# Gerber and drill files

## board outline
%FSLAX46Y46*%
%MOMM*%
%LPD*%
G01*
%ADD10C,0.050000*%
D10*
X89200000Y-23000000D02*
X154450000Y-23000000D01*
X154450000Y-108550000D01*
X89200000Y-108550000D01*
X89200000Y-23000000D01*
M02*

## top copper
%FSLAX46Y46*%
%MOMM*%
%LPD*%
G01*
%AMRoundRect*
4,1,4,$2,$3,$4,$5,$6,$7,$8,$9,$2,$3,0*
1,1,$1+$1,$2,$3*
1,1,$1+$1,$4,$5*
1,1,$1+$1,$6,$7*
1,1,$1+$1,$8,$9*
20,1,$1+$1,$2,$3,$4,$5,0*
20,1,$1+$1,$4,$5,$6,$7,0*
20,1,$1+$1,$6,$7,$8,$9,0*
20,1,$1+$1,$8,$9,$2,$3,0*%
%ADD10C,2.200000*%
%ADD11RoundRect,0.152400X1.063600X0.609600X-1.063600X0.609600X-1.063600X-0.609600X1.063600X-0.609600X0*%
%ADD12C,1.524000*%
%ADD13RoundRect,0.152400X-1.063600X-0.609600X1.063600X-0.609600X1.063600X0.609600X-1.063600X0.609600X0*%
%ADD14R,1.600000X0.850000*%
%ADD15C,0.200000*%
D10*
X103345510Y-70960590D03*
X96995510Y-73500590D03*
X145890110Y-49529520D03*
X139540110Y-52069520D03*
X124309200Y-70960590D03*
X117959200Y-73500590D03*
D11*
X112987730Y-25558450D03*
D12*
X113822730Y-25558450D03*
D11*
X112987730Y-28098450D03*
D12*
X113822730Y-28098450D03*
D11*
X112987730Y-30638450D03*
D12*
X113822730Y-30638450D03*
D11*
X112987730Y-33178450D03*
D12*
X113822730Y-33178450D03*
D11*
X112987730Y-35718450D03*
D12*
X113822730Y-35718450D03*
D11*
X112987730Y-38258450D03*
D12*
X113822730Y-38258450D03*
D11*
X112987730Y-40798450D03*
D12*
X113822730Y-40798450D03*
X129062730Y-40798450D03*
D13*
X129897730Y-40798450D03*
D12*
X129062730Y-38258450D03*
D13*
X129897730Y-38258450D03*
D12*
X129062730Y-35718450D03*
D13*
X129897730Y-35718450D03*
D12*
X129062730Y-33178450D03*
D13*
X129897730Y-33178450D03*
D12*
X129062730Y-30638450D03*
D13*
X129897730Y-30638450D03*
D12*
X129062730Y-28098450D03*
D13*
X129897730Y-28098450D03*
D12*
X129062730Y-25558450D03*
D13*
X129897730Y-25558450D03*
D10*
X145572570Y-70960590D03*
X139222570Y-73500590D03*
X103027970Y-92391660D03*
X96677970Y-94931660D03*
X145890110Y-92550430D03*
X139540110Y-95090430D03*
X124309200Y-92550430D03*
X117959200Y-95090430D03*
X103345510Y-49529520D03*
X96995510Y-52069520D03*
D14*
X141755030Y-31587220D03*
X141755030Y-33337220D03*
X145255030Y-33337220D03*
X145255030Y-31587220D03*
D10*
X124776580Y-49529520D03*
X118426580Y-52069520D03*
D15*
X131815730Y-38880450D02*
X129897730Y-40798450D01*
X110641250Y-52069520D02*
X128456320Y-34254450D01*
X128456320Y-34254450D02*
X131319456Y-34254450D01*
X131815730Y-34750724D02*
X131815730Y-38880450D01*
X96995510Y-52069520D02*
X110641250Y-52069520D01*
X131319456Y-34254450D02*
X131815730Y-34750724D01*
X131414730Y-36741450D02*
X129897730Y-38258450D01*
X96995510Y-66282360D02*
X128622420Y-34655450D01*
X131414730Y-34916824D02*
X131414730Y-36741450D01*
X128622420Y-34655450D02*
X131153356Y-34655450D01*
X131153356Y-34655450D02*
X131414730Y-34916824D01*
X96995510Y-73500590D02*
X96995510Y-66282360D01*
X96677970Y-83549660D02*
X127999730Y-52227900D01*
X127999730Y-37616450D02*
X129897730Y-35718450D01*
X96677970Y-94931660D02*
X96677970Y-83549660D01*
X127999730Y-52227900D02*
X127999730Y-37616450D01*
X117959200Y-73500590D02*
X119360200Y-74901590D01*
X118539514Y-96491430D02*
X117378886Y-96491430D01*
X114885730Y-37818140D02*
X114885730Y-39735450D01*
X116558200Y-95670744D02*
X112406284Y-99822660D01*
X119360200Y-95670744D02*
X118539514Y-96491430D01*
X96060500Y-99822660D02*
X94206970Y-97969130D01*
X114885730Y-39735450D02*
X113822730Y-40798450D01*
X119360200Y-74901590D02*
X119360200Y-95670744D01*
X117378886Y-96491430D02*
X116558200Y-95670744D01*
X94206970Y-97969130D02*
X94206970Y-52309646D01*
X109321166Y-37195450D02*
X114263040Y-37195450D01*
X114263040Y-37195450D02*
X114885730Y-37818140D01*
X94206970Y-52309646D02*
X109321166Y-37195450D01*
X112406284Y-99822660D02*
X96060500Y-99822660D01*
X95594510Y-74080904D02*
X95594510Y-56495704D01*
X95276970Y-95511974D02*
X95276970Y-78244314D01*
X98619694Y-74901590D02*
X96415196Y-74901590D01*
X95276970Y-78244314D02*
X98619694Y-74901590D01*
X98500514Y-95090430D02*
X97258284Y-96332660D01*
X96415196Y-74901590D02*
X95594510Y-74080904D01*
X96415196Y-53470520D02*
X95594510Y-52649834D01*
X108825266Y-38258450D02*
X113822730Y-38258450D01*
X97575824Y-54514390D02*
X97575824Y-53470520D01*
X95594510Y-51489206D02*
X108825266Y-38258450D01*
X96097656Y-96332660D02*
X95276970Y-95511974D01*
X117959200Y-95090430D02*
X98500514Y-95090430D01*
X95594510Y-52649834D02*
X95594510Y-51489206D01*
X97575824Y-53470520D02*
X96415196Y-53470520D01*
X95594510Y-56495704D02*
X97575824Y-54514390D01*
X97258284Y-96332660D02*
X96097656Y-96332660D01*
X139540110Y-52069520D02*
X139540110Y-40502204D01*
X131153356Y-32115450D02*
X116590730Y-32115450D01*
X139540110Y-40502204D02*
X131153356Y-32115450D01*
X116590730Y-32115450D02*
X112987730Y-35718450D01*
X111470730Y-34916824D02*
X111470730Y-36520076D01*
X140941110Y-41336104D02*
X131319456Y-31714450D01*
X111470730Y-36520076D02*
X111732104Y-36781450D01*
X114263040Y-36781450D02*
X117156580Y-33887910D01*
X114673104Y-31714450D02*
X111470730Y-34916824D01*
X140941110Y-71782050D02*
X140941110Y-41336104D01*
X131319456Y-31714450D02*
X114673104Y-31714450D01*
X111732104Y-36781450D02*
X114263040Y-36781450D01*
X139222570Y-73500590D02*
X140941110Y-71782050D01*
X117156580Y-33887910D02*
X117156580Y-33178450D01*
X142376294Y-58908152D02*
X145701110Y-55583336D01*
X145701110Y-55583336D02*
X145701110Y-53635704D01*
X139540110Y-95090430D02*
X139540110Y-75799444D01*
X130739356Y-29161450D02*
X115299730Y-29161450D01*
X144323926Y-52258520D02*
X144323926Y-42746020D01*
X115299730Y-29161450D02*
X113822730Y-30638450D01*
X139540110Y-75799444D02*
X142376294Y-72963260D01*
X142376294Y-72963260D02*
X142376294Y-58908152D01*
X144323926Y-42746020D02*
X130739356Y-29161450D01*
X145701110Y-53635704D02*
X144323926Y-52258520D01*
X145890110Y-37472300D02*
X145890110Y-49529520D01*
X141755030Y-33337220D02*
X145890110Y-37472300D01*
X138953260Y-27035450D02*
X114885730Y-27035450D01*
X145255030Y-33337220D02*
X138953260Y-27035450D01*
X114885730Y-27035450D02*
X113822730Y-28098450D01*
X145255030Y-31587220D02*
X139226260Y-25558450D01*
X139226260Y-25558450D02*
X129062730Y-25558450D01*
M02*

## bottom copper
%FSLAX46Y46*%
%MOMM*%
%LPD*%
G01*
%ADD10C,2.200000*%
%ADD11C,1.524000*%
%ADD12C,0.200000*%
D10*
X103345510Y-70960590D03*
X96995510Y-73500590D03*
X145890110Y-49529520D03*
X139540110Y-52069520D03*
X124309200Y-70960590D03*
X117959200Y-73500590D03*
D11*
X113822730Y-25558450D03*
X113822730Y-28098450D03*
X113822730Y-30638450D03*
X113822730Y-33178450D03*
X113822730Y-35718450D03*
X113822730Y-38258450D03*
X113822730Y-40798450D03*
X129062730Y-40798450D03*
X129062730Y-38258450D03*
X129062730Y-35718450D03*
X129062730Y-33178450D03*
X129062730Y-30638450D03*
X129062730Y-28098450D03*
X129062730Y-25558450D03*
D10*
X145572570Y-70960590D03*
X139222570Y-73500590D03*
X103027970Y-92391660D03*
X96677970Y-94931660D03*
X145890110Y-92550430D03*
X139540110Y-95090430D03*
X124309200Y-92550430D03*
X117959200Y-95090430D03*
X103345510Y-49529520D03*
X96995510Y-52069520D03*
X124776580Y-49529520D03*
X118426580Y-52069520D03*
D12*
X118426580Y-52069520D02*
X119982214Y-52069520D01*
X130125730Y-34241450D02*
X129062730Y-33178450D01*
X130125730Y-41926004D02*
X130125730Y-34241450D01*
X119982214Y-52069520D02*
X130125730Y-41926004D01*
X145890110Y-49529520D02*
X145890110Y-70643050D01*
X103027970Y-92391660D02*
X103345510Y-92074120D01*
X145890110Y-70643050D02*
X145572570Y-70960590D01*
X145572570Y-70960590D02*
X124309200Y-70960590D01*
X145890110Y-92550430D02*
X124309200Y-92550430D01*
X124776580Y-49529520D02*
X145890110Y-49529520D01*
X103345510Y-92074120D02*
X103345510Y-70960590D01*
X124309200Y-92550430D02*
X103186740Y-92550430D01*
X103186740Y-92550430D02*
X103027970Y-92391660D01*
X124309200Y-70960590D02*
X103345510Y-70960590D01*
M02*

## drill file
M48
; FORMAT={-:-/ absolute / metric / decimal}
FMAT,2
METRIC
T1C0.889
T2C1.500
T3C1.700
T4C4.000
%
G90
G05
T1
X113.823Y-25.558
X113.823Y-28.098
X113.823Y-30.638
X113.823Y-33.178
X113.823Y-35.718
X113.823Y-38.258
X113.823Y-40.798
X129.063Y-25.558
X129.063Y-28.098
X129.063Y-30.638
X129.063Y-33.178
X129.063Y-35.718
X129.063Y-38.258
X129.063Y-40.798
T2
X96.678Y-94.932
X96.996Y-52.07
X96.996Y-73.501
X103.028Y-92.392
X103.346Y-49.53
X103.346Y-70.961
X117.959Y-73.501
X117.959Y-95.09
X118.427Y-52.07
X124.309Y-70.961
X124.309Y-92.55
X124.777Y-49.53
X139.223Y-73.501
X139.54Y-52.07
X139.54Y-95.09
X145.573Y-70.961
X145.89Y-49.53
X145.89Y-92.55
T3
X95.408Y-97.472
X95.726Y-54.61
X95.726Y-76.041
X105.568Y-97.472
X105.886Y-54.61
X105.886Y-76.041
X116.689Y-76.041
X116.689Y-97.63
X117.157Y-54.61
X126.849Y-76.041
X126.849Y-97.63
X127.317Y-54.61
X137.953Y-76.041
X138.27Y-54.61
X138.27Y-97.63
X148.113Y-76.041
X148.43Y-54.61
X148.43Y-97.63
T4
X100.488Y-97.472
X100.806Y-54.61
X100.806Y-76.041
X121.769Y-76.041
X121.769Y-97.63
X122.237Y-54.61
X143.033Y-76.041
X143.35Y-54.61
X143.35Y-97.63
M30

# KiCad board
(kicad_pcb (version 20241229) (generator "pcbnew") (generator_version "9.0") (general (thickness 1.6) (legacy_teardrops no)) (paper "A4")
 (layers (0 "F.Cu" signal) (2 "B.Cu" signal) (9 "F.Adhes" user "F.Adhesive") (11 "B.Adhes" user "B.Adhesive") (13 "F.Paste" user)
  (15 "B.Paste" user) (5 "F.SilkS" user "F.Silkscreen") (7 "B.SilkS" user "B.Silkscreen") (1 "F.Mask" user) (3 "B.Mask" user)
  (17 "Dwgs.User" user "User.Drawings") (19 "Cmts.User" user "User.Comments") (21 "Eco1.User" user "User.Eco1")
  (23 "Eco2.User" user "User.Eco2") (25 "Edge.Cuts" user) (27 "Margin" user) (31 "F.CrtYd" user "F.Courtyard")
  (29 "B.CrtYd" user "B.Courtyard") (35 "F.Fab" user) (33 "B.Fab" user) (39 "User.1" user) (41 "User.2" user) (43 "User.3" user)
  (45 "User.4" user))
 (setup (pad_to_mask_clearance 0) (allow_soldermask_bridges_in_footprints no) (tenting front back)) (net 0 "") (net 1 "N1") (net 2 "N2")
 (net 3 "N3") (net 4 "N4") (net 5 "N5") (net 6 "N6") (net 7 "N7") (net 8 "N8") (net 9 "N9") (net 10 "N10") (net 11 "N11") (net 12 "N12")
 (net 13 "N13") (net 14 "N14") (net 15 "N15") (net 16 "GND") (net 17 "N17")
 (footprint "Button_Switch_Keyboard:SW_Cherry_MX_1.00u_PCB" (layer "F.Cu") (at 103.34551 70.96059)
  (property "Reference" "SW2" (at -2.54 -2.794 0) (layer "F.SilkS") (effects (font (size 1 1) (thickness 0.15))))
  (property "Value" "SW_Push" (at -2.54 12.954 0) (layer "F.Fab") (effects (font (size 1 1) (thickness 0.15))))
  (pad "" np_thru_hole circle (at -7.62 5.08) (size 1.7 1.7) (drill 1.7) (layers "*.Cu" "*.Mask"))
  (pad "" np_thru_hole circle (at -2.54 5.08) (size 4 4) (drill 4) (layers "*.Cu" "*.Mask"))
  (pad "" np_thru_hole circle (at 2.54 5.08) (size 1.7 1.7) (drill 1.7) (layers "*.Cu" "*.Mask"))
  (pad "1" thru_hole circle (at 0 0) (size 2.2 2.2) (drill 1.5) (layers "*.Cu" "*.Mask") (remove_unused_layers no) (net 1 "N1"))
  (pad "2" thru_hole circle (at -6.35 2.54) (size 2.2 2.2) (drill 1.5) (layers "*.Cu" "*.Mask") (remove_unused_layers no) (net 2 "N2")))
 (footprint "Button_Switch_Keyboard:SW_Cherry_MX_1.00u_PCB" (layer "F.Cu") (at 145.89011 49.52952)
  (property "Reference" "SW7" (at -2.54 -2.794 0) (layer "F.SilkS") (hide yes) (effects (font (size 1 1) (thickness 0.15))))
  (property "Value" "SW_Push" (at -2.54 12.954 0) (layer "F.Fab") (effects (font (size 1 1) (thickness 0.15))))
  (pad "" np_thru_hole circle (at -7.62 5.08) (size 1.7 1.7) (drill 1.7) (layers "*.Cu" "*.Mask"))
  (pad "" np_thru_hole circle (at -2.54 5.08) (size 4 4) (drill 4) (layers "*.Cu" "*.Mask"))
  (pad "" np_thru_hole circle (at 2.54 5.08) (size 1.7 1.7) (drill 1.7) (layers "*.Cu" "*.Mask"))
  (pad "1" thru_hole circle (at 0 0) (size 2.2 2.2) (drill 1.5) (layers "*.Cu" "*.Mask") (remove_unused_layers no) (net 1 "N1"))
  (pad "2" thru_hole circle (at -6.35 2.54) (size 2.2 2.2) (drill 1.5) (layers "*.Cu" "*.Mask") (remove_unused_layers no) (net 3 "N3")))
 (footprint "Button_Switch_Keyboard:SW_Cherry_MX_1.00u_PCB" (layer "F.Cu") (at 124.3092 70.96059)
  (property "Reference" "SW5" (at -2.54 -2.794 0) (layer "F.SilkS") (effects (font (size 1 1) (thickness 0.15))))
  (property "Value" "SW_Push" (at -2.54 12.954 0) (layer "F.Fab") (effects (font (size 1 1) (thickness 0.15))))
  (pad "" np_thru_hole circle (at -7.62 5.08) (size 1.7 1.7) (drill 1.7) (layers "*.Cu" "*.Mask"))
  (pad "" np_thru_hole circle (at -2.54 5.08) (size 4 4) (drill 4) (layers "*.Cu" "*.Mask"))
  (pad "" np_thru_hole circle (at 2.54 5.08) (size 1.7 1.7) (drill 1.7) (layers "*.Cu" "*.Mask"))
  (pad "1" thru_hole circle (at 0 0) (size 2.2 2.2) (drill 1.5) (layers "*.Cu" "*.Mask") (remove_unused_layers no) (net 1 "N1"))
  (pad "2" thru_hole circle (at -6.35 2.54) (size 2.2 2.2) (drill 1.5) (layers "*.Cu" "*.Mask") (remove_unused_layers no) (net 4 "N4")))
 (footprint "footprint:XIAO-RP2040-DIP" (layer "F.Cu") (at 121.44273 33.17845)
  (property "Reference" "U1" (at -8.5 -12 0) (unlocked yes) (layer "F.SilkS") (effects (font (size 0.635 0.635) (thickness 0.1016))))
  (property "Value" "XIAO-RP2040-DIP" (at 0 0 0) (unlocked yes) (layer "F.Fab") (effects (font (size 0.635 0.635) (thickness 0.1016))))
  (pad "1" smd roundrect (at -8.455 -7.62 180) (size 2.432 1.524) (layers "F.Cu" "F.Mask") (roundrect_rratio 0.1) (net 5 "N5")
   (thermal_bridge_angle 45))
  (pad "1" thru_hole circle (at -7.62 -7.62 180) (size 1.524 1.524) (drill 0.889) (layers "*.Cu" "*.Mask") (remove_unused_layers no)
   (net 5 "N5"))
  (pad "2" smd roundrect (at -8.455 -5.08 180) (size 2.432 1.524) (layers "F.Cu" "F.Mask") (roundrect_rratio 0.1) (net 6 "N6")
   (thermal_bridge_angle 45))
  (pad "2" thru_hole circle (at -7.62 -5.08 180) (size 1.524 1.524) (drill 0.889) (layers "*.Cu" "*.Mask") (remove_unused_layers no)
   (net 6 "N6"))
  (pad "3" smd roundrect (at -8.455 -2.54 180) (size 2.432 1.524) (layers "F.Cu" "F.Mask") (roundrect_rratio 0.1) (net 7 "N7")
   (thermal_bridge_angle 45))
  (pad "3" thru_hole circle (at -7.62 -2.54 180) (size 1.524 1.524) (drill 0.889) (layers "*.Cu" "*.Mask") (remove_unused_layers no)
   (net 7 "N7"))
  (pad "4" smd roundrect (at -8.455 0 180) (size 2.432 1.524) (layers "F.Cu" "F.Mask") (roundrect_rratio 0.1) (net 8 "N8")
   (thermal_bridge_angle 45))
  (pad "4" thru_hole circle (at -7.62 0 180) (size 1.524 1.524) (drill 0.889) (layers "*.Cu" "*.Mask") (remove_unused_layers no)
   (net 8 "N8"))
  (pad "5" smd roundrect (at -8.455 2.54 180) (size 2.432 1.524) (layers "F.Cu" "F.Mask") (roundrect_rratio 0.1) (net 3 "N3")
   (thermal_bridge_angle 45))
  (pad "5" thru_hole circle (at -7.62 2.54 180) (size 1.524 1.524) (drill 0.889) (layers "*.Cu" "*.Mask") (remove_unused_layers no)
   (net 3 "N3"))
  (pad "6" smd roundrect (at -8.455 5.08 180) (size 2.432 1.524) (layers "F.Cu" "F.Mask") (roundrect_rratio 0.1) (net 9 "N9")
   (thermal_bridge_angle 45))
  (pad "6" thru_hole circle (at -7.62 5.08 180) (size 1.524 1.524) (drill 0.889) (layers "*.Cu" "*.Mask") (remove_unused_layers no)
   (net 9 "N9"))
  (pad "7" smd roundrect (at -8.455 7.62 180) (size 2.432 1.524) (layers "F.Cu" "F.Mask") (roundrect_rratio 0.1) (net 4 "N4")
   (thermal_bridge_angle 45))
  (pad "7" thru_hole circle (at -7.62 7.62 180) (size 1.524 1.524) (drill 0.889) (layers "*.Cu" "*.Mask") (remove_unused_layers no)
   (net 4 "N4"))
  (pad "8" thru_hole circle (at 7.62 7.62) (size 1.524 1.524) (drill 0.889) (layers "*.Cu" "*.Mask") (remove_unused_layers no)
   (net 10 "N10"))
  (pad "8" smd roundrect (at 8.455 7.62) (size 2.432 1.524) (layers "F.Cu" "F.Mask") (roundrect_rratio 0.1) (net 10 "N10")
   (thermal_bridge_angle 45))
  (pad "9" thru_hole circle (at 7.62 5.08) (size 1.524 1.524) (drill 0.889) (layers "*.Cu" "*.Mask") (remove_unused_layers no) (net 2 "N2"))
  (pad "9" smd roundrect (at 8.455 5.08) (size 2.432 1.524) (layers "F.Cu" "F.Mask") (roundrect_rratio 0.1) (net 2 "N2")
   (thermal_bridge_angle 45))
  (pad "10" thru_hole circle (at 7.62 2.54) (size 1.524 1.524) (drill 0.889) (layers "*.Cu" "*.Mask") (remove_unused_layers no)
   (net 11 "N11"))
  (pad "10" smd roundrect (at 8.455 2.54) (size 2.432 1.524) (layers "F.Cu" "F.Mask") (roundrect_rratio 0.1) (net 11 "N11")
   (thermal_bridge_angle 45))
  (pad "11" thru_hole circle (at 7.62 0) (size 1.524 1.524) (drill 0.889) (layers "*.Cu" "*.Mask") (remove_unused_layers no) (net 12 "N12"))
  (pad "11" smd roundrect (at 8.455 0) (size 2.432 1.524) (layers "F.Cu" "F.Mask") (roundrect_rratio 0.1) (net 12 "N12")
   (thermal_bridge_angle 45))
  (pad "12" thru_hole circle (at 7.62 -2.54) (size 1.524 1.524) (drill 0.889) (layers "*.Cu" "*.Mask") (remove_unused_layers no)
   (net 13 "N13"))
  (pad "12" smd roundrect (at 8.455 -2.54) (size 2.432 1.524) (layers "F.Cu" "F.Mask") (roundrect_rratio 0.1) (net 13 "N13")
   (thermal_bridge_angle 45))
  (pad "13" thru_hole circle (at 7.62 -5.08) (size 1.524 1.524) (drill 0.889) (layers "*.Cu" "*.Mask") (remove_unused_layers no)
   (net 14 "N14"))
  (pad "13" smd roundrect (at 8.455 -5.08) (size 2.432 1.524) (layers "F.Cu" "F.Mask") (roundrect_rratio 0.1) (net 14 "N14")
   (thermal_bridge_angle 45))
  (pad "14" thru_hole circle (at 7.62 -7.62) (size 1.524 1.524) (drill 0.889) (layers "*.Cu" "*.Mask") (remove_unused_layers no)
   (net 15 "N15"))
  (pad "14" smd roundrect (at 8.455 -7.62) (size 2.432 1.524) (layers "F.Cu" "F.Mask") (roundrect_rratio 0.1) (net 15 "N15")
   (thermal_bridge_angle 45)))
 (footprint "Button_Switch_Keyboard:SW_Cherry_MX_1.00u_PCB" (layer "F.Cu") (at 145.57257 70.96059)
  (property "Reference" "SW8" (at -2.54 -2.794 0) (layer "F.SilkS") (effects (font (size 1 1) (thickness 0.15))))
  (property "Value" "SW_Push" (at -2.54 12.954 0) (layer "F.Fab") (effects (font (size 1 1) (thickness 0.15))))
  (pad "" np_thru_hole circle (at -7.62 5.08) (size 1.7 1.7) (drill 1.7) (layers "*.Cu" "*.Mask"))
  (pad "" np_thru_hole circle (at -2.54 5.08) (size 4 4) (drill 4) (layers "*.Cu" "*.Mask"))
  (pad "" np_thru_hole circle (at 2.54 5.08) (size 1.7 1.7) (drill 1.7) (layers "*.Cu" "*.Mask"))
  (pad "1" thru_hole circle (at 0 0) (size 2.2 2.2) (drill 1.5) (layers "*.Cu" "*.Mask") (remove_unused_layers no) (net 1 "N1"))
  (pad "2" thru_hole circle (at -6.35 2.54) (size 2.2 2.2) (drill 1.5) (layers "*.Cu" "*.Mask") (remove_unused_layers no) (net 8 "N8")))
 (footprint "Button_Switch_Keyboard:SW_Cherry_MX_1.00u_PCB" (layer "F.Cu") (at 103.02797 92.39166)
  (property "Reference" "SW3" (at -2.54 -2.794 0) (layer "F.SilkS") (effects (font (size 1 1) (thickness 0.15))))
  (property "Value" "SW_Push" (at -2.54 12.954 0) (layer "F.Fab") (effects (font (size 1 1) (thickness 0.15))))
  (pad "" np_thru_hole circle (at -7.62 5.08) (size 1.7 1.7) (drill 1.7) (layers "*.Cu" "*.Mask"))
  (pad "" np_thru_hole circle (at -2.54 5.08) (size 4 4) (drill 4) (layers "*.Cu" "*.Mask"))
  (pad "" np_thru_hole circle (at 2.54 5.08) (size 1.7 1.7) (drill 1.7) (layers "*.Cu" "*.Mask"))
  (pad "1" thru_hole circle (at 0 0) (size 2.2 2.2) (drill 1.5) (layers "*.Cu" "*.Mask") (remove_unused_layers no) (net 1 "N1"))
  (pad "2" thru_hole circle (at -6.35 2.54) (size 2.2 2.2) (drill 1.5) (layers "*.Cu" "*.Mask") (remove_unused_layers no) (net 11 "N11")))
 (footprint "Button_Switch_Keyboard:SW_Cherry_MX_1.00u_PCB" (layer "F.Cu") (at 145.89011 92.55043)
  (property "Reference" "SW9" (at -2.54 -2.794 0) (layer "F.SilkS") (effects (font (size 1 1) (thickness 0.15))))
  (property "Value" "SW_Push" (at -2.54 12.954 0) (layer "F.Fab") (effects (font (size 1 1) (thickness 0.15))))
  (pad "" np_thru_hole circle (at -7.62 5.08) (size 1.7 1.7) (drill 1.7) (layers "*.Cu" "*.Mask"))
  (pad "" np_thru_hole circle (at -2.54 5.08) (size 4 4) (drill 4) (layers "*.Cu" "*.Mask"))
  (pad "" np_thru_hole circle (at 2.54 5.08) (size 1.7 1.7) (drill 1.7) (layers "*.Cu" "*.Mask"))
  (pad "1" thru_hole circle (at 0 0) (size 2.2 2.2) (drill 1.5) (layers "*.Cu" "*.Mask") (remove_unused_layers no) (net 1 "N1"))
  (pad "2" thru_hole circle (at -6.35 2.54) (size 2.2 2.2) (drill 1.5) (layers "*.Cu" "*.Mask") (remove_unused_layers no) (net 7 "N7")))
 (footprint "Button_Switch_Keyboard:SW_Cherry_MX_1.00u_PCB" (layer "F.Cu") (at 124.3092 92.55043)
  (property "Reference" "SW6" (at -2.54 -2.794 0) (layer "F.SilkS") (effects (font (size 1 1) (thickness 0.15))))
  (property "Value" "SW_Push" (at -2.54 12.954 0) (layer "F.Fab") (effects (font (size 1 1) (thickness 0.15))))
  (pad "" np_thru_hole circle (at -7.62 5.08) (size 1.7 1.7) (drill 1.7) (layers "*.Cu" "*.Mask"))
  (pad "" np_thru_hole circle (at -2.54 5.08) (size 4 4) (drill 4) (layers "*.Cu" "*.Mask"))
  (pad "" np_thru_hole circle (at 2.54 5.08) (size 1.7 1.7) (drill 1.7) (layers "*.Cu" "*.Mask"))
  (pad "1" thru_hole circle (at 0 0) (size 2.2 2.2) (drill 1.5) (layers "*.Cu" "*.Mask") (remove_unused_layers no) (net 1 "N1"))
  (pad "2" thru_hole circle (at -6.35 2.54) (size 2.2 2.2) (drill 1.5) (layers "*.Cu" "*.Mask") (remove_unused_layers no) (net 9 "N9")))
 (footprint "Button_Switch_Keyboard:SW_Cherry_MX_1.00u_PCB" (layer "F.Cu") (at 103.34551 49.52952)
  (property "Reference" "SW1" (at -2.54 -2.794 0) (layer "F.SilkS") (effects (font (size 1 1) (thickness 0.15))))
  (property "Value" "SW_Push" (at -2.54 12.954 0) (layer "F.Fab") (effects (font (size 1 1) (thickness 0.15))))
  (pad "" np_thru_hole circle (at -7.62 5.08) (size 1.7 1.7) (drill 1.7) (layers "*.Cu" "*.Mask"))
  (pad "" np_thru_hole circle (at -2.54 5.08) (size 4 4) (drill 4) (layers "*.Cu" "*.Mask"))
  (pad "" np_thru_hole circle (at 2.54 5.08) (size 1.7 1.7) (drill 1.7) (layers "*.Cu" "*.Mask"))
  (pad "1" thru_hole circle (at 0 0) (size 2.2 2.2) (drill 1.5) (layers "*.Cu" "*.Mask") (remove_unused_layers no) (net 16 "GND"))
  (pad "2" thru_hole circle (at -6.35 2.54) (size 2.2 2.2) (drill 1.5) (layers "*.Cu" "*.Mask") (remove_unused_layers no) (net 10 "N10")))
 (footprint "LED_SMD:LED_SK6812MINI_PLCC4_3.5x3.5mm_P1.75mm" (layer "F.Cu") (at 143.50503 32.46222)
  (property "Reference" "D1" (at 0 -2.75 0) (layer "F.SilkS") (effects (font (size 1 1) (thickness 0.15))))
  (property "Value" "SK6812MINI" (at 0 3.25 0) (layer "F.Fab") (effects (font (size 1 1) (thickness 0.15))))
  (pad "1" smd rect (at -1.75 -0.875) (size 1.6 0.85) (layers "F.Cu" "F.Mask" "F.Paste") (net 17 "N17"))
  (pad "2" smd rect (at -1.75 0.875) (size 1.6 0.85) (layers "F.Cu" "F.Mask" "F.Paste") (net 1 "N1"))
  (pad "3" smd rect (at 1.75 0.875) (size 1.6 0.85) (layers "F.Cu" "F.Mask" "F.Paste") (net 6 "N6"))
  (pad "4" smd rect (at 1.75 -0.875) (size 1.6 0.85) (layers "F.Cu" "F.Mask" "F.Paste") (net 15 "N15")))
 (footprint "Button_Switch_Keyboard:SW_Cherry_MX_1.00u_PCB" (layer "F.Cu") (at 124.77658 49.52952)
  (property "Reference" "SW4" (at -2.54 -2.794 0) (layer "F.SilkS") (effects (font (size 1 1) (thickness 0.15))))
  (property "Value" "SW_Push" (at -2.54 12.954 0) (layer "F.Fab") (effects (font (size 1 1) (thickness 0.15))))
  (pad "" np_thru_hole circle (at -7.62 5.08) (size 1.7 1.7) (drill 1.7) (layers "*.Cu" "*.Mask"))
  (pad "" np_thru_hole circle (at -2.54 5.08) (size 4 4) (drill 4) (layers "*.Cu" "*.Mask"))
  (pad "" np_thru_hole circle (at 2.54 5.08) (size 1.7 1.7) (drill 1.7) (layers "*.Cu" "*.Mask"))
  (pad "1" thru_hole circle (at 0 0) (size 2.2 2.2) (drill 1.5) (layers "*.Cu" "*.Mask") (remove_unused_layers no) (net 1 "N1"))
  (pad "2" thru_hole circle (at -6.35 2.54) (size 2.2 2.2) (drill 1.5) (layers "*.Cu" "*.Mask") (remove_unused_layers no) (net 12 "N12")))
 (gr_rect (start 89.2 23) (end 154.45 108.55) (stroke (width 0.05) (type default)) (fill no) (layer "Edge.Cuts"))
 (segment (start 131.81573 38.88045) (end 129.89773 40.79845) (width 0.2) (layer "F.Cu") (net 10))
 (segment (start 110.64125 52.06952) (end 128.45632 34.25445) (width 0.2) (layer "F.Cu") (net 10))
 (segment (start 128.45632 34.25445) (end 131.319456 34.25445) (width 0.2) (layer "F.Cu") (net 10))
 (segment (start 131.81573 34.750724) (end 131.81573 38.88045) (width 0.2) (layer "F.Cu") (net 10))
 (segment (start 96.99551 52.06952) (end 110.64125 52.06952) (width 0.2) (layer "F.Cu") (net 10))
 (segment (start 131.319456 34.25445) (end 131.81573 34.750724) (width 0.2) (layer "F.Cu") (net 10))
 (segment (start 131.41473 36.74145) (end 129.89773 38.25845) (width 0.2) (layer "F.Cu") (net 2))
 (segment (start 96.99551 66.28236) (end 128.62242 34.65545) (width 0.2) (layer "F.Cu") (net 2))
 (segment (start 131.41473 34.916824) (end 131.41473 36.74145) (width 0.2) (layer "F.Cu") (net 2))
 (segment (start 128.62242 34.65545) (end 131.153356 34.65545) (width 0.2) (layer "F.Cu") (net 2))
 (segment (start 131.153356 34.65545) (end 131.41473 34.916824) (width 0.2) (layer "F.Cu") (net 2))
 (segment (start 96.99551 73.50059) (end 96.99551 66.28236) (width 0.2) (layer "F.Cu") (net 2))
 (segment (start 96.67797 83.54966) (end 127.99973 52.2279) (width 0.2) (layer "F.Cu") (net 11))
 (segment (start 127.99973 37.61645) (end 129.89773 35.71845) (width 0.2) (layer "F.Cu") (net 11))
 (segment (start 96.67797 94.93166) (end 96.67797 83.54966) (width 0.2) (layer "F.Cu") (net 11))
 (segment (start 127.99973 52.2279) (end 127.99973 37.61645) (width 0.2) (layer "F.Cu") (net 11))
 (segment (start 118.42658 52.06952) (end 119.982214 52.06952) (width 0.2) (layer "B.Cu") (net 12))
 (segment (start 130.12573 34.24145) (end 129.06273 33.17845) (width 0.2) (layer "B.Cu") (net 12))
 (segment (start 130.12573 41.926004) (end 130.12573 34.24145) (width 0.2) (layer "B.Cu") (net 12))
 (segment (start 119.982214 52.06952) (end 130.12573 41.926004) (width 0.2) (layer "B.Cu") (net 12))
 (segment (start 117.9592 73.50059) (end 119.3602 74.90159) (width 0.2) (layer "F.Cu") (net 4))
 (segment (start 118.539514 96.49143) (end 117.378886 96.49143) (width 0.2) (layer "F.Cu") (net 4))
 (segment (start 114.88573 37.81814) (end 114.88573 39.73545) (width 0.2) (layer "F.Cu") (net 4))
 (segment (start 116.5582 95.670744) (end 112.406284 99.82266) (width 0.2) (layer "F.Cu") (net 4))
 (segment (start 119.3602 95.670744) (end 118.539514 96.49143) (width 0.2) (layer "F.Cu") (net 4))
 (segment (start 96.0605 99.82266) (end 94.20697 97.96913) (width 0.2) (layer "F.Cu") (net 4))
 (segment (start 114.88573 39.73545) (end 113.82273 40.79845) (width 0.2) (layer "F.Cu") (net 4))
 (segment (start 119.3602 74.90159) (end 119.3602 95.670744) (width 0.2) (layer "F.Cu") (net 4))
 (segment (start 117.378886 96.49143) (end 116.5582 95.670744) (width 0.2) (layer "F.Cu") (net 4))
 (segment (start 94.20697 97.96913) (end 94.20697 52.309646) (width 0.2) (layer "F.Cu") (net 4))
 (segment (start 109.321166 37.19545) (end 114.26304 37.19545) (width 0.2) (layer "F.Cu") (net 4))
 (segment (start 114.26304 37.19545) (end 114.88573 37.81814) (width 0.2) (layer "F.Cu") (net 4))
 (segment (start 94.20697 52.309646) (end 109.321166 37.19545) (width 0.2) (layer "F.Cu") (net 4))
 (segment (start 112.406284 99.82266) (end 96.0605 99.82266) (width 0.2) (layer "F.Cu") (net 4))
 (segment (start 95.59451 74.080904) (end 95.59451 56.495704) (width 0.2) (layer "F.Cu") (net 9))
 (segment (start 95.27697 95.511974) (end 95.27697 78.244314) (width 0.2) (layer "F.Cu") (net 9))
 (segment (start 98.619694 74.90159) (end 96.415196 74.90159) (width 0.2) (layer "F.Cu") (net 9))
 (segment (start 95.27697 78.244314) (end 98.619694 74.90159) (width 0.2) (layer "F.Cu") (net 9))
 (segment (start 98.500514 95.09043) (end 97.258284 96.33266) (width 0.2) (layer "F.Cu") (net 9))
 (segment (start 96.415196 74.90159) (end 95.59451 74.080904) (width 0.2) (layer "F.Cu") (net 9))
 (segment (start 96.415196 53.47052) (end 95.59451 52.649834) (width 0.2) (layer "F.Cu") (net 9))
 (segment (start 108.825266 38.25845) (end 113.82273 38.25845) (width 0.2) (layer "F.Cu") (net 9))
 (segment (start 97.575824 54.51439) (end 97.575824 53.47052) (width 0.2) (layer "F.Cu") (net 9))
 (segment (start 95.59451 51.489206) (end 108.825266 38.25845) (width 0.2) (layer "F.Cu") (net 9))
 (segment (start 96.097656 96.33266) (end 95.27697 95.511974) (width 0.2) (layer "F.Cu") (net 9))
 (segment (start 117.9592 95.09043) (end 98.500514 95.09043) (width 0.2) (layer "F.Cu") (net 9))
 (segment (start 95.59451 52.649834) (end 95.59451 51.489206) (width 0.2) (layer "F.Cu") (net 9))
 (segment (start 97.575824 53.47052) (end 96.415196 53.47052) (width 0.2) (layer "F.Cu") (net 9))
 (segment (start 95.59451 56.495704) (end 97.575824 54.51439) (width 0.2) (layer "F.Cu") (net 9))
 (segment (start 97.258284 96.33266) (end 96.097656 96.33266) (width 0.2) (layer "F.Cu") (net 9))
 (segment (start 139.54011 52.06952) (end 139.54011 40.502204) (width 0.2) (layer "F.Cu") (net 3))
 (segment (start 131.153356 32.11545) (end 116.59073 32.11545) (width 0.2) (layer "F.Cu") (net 3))
 (segment (start 139.54011 40.502204) (end 131.153356 32.11545) (width 0.2) (layer "F.Cu") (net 3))
 (segment (start 116.59073 32.11545) (end 112.98773 35.71845) (width 0.2) (layer "F.Cu") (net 3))
 (segment (start 111.47073 34.916824) (end 111.47073 36.520076) (width 0.2) (layer "F.Cu") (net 8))
 (segment (start 140.94111 41.336104) (end 131.319456 31.71445) (width 0.2) (layer "F.Cu") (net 8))
 (segment (start 111.47073 36.520076) (end 111.732104 36.78145) (width 0.2) (layer "F.Cu") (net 8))
 (segment (start 114.26304 36.78145) (end 117.15658 33.88791) (width 0.2) (layer "F.Cu") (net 8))
 (segment (start 114.673104 31.71445) (end 111.47073 34.916824) (width 0.2) (layer "F.Cu") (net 8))
 (segment (start 140.94111 71.78205) (end 140.94111 41.336104) (width 0.2) (layer "F.Cu") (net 8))
 (segment (start 131.319456 31.71445) (end 114.673104 31.71445) (width 0.2) (layer "F.Cu") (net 8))
 (segment (start 111.732104 36.78145) (end 114.26304 36.78145) (width 0.2) (layer "F.Cu") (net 8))
 (segment (start 139.22257 73.50059) (end 140.94111 71.78205) (width 0.2) (layer "F.Cu") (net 8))
 (segment (start 117.15658 33.88791) (end 117.15658 33.17845) (width 0.2) (layer "F.Cu") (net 8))
 (segment (start 142.376294 58.908152) (end 145.70111 55.583336) (width 0.2) (layer "F.Cu") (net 7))
 (segment (start 145.70111 55.583336) (end 145.70111 53.635704) (width 0.2) (layer "F.Cu") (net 7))
 (segment (start 139.54011 95.09043) (end 139.54011 75.799444) (width 0.2) (layer "F.Cu") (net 7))
 (segment (start 130.739356 29.16145) (end 115.29973 29.16145) (width 0.2) (layer "F.Cu") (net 7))
 (segment (start 144.323926 52.25852) (end 144.323926 42.74602) (width 0.2) (layer "F.Cu") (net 7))
 (segment (start 115.29973 29.16145) (end 113.82273 30.63845) (width 0.2) (layer "F.Cu") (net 7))
 (segment (start 139.54011 75.799444) (end 142.376294 72.96326) (width 0.2) (layer "F.Cu") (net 7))
 (segment (start 142.376294 72.96326) (end 142.376294 58.908152) (width 0.2) (layer "F.Cu") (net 7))
 (segment (start 144.323926 42.74602) (end 130.739356 29.16145) (width 0.2) (layer "F.Cu") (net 7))
 (segment (start 145.70111 53.635704) (end 144.323926 52.25852) (width 0.2) (layer "F.Cu") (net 7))
 (segment (start 145.89011 37.4723) (end 145.89011 49.52952) (width 0.2) (layer "F.Cu") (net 1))
 (segment (start 141.75503 33.33722) (end 145.89011 37.4723) (width 0.2) (layer "F.Cu") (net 1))
 (segment (start 145.89011 49.52952) (end 145.89011 70.64305) (width 0.2) (layer "B.Cu") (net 1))
 (segment (start 103.02797 92.39166) (end 103.34551 92.07412) (width 0.2) (layer "B.Cu") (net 1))
 (segment (start 145.89011 70.64305) (end 145.57257 70.96059) (width 0.2) (layer "B.Cu") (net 1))
 (segment (start 145.57257 70.96059) (end 124.3092 70.96059) (width 0.2) (layer "B.Cu") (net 1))
 (segment (start 145.89011 92.55043) (end 124.3092 92.55043) (width 0.2) (layer "B.Cu") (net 1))
 (segment (start 124.77658 49.52952) (end 145.89011 49.52952) (width 0.2) (layer "B.Cu") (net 1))
 (segment (start 103.34551 92.07412) (end 103.34551 70.96059) (width 0.2) (layer "B.Cu") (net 1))
 (segment (start 124.3092 92.55043) (end 103.18674 92.55043) (width 0.2) (layer "B.Cu") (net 1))
 (segment (start 103.18674 92.55043) (end 103.02797 92.39166) (width 0.2) (layer "B.Cu") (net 1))
 (segment (start 124.3092 70.96059) (end 103.34551 70.96059) (width 0.2) (layer "B.Cu") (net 1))
 (segment (start 138.95326 27.03545) (end 114.88573 27.03545) (width 0.2) (layer "F.Cu") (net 6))
 (segment (start 145.25503 33.33722) (end 138.95326 27.03545) (width 0.2) (layer "F.Cu") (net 6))
 (segment (start 114.88573 27.03545) (end 113.82273 28.09845) (width 0.2) (layer "F.Cu") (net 6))
 (segment (start 145.25503 31.58722) (end 139.22626 25.55845) (width 0.2) (layer "F.Cu") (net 15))
 (segment (start 139.22626 25.55845) (end 129.06273 25.55845) (width 0.2) (layer "F.Cu") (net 15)))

